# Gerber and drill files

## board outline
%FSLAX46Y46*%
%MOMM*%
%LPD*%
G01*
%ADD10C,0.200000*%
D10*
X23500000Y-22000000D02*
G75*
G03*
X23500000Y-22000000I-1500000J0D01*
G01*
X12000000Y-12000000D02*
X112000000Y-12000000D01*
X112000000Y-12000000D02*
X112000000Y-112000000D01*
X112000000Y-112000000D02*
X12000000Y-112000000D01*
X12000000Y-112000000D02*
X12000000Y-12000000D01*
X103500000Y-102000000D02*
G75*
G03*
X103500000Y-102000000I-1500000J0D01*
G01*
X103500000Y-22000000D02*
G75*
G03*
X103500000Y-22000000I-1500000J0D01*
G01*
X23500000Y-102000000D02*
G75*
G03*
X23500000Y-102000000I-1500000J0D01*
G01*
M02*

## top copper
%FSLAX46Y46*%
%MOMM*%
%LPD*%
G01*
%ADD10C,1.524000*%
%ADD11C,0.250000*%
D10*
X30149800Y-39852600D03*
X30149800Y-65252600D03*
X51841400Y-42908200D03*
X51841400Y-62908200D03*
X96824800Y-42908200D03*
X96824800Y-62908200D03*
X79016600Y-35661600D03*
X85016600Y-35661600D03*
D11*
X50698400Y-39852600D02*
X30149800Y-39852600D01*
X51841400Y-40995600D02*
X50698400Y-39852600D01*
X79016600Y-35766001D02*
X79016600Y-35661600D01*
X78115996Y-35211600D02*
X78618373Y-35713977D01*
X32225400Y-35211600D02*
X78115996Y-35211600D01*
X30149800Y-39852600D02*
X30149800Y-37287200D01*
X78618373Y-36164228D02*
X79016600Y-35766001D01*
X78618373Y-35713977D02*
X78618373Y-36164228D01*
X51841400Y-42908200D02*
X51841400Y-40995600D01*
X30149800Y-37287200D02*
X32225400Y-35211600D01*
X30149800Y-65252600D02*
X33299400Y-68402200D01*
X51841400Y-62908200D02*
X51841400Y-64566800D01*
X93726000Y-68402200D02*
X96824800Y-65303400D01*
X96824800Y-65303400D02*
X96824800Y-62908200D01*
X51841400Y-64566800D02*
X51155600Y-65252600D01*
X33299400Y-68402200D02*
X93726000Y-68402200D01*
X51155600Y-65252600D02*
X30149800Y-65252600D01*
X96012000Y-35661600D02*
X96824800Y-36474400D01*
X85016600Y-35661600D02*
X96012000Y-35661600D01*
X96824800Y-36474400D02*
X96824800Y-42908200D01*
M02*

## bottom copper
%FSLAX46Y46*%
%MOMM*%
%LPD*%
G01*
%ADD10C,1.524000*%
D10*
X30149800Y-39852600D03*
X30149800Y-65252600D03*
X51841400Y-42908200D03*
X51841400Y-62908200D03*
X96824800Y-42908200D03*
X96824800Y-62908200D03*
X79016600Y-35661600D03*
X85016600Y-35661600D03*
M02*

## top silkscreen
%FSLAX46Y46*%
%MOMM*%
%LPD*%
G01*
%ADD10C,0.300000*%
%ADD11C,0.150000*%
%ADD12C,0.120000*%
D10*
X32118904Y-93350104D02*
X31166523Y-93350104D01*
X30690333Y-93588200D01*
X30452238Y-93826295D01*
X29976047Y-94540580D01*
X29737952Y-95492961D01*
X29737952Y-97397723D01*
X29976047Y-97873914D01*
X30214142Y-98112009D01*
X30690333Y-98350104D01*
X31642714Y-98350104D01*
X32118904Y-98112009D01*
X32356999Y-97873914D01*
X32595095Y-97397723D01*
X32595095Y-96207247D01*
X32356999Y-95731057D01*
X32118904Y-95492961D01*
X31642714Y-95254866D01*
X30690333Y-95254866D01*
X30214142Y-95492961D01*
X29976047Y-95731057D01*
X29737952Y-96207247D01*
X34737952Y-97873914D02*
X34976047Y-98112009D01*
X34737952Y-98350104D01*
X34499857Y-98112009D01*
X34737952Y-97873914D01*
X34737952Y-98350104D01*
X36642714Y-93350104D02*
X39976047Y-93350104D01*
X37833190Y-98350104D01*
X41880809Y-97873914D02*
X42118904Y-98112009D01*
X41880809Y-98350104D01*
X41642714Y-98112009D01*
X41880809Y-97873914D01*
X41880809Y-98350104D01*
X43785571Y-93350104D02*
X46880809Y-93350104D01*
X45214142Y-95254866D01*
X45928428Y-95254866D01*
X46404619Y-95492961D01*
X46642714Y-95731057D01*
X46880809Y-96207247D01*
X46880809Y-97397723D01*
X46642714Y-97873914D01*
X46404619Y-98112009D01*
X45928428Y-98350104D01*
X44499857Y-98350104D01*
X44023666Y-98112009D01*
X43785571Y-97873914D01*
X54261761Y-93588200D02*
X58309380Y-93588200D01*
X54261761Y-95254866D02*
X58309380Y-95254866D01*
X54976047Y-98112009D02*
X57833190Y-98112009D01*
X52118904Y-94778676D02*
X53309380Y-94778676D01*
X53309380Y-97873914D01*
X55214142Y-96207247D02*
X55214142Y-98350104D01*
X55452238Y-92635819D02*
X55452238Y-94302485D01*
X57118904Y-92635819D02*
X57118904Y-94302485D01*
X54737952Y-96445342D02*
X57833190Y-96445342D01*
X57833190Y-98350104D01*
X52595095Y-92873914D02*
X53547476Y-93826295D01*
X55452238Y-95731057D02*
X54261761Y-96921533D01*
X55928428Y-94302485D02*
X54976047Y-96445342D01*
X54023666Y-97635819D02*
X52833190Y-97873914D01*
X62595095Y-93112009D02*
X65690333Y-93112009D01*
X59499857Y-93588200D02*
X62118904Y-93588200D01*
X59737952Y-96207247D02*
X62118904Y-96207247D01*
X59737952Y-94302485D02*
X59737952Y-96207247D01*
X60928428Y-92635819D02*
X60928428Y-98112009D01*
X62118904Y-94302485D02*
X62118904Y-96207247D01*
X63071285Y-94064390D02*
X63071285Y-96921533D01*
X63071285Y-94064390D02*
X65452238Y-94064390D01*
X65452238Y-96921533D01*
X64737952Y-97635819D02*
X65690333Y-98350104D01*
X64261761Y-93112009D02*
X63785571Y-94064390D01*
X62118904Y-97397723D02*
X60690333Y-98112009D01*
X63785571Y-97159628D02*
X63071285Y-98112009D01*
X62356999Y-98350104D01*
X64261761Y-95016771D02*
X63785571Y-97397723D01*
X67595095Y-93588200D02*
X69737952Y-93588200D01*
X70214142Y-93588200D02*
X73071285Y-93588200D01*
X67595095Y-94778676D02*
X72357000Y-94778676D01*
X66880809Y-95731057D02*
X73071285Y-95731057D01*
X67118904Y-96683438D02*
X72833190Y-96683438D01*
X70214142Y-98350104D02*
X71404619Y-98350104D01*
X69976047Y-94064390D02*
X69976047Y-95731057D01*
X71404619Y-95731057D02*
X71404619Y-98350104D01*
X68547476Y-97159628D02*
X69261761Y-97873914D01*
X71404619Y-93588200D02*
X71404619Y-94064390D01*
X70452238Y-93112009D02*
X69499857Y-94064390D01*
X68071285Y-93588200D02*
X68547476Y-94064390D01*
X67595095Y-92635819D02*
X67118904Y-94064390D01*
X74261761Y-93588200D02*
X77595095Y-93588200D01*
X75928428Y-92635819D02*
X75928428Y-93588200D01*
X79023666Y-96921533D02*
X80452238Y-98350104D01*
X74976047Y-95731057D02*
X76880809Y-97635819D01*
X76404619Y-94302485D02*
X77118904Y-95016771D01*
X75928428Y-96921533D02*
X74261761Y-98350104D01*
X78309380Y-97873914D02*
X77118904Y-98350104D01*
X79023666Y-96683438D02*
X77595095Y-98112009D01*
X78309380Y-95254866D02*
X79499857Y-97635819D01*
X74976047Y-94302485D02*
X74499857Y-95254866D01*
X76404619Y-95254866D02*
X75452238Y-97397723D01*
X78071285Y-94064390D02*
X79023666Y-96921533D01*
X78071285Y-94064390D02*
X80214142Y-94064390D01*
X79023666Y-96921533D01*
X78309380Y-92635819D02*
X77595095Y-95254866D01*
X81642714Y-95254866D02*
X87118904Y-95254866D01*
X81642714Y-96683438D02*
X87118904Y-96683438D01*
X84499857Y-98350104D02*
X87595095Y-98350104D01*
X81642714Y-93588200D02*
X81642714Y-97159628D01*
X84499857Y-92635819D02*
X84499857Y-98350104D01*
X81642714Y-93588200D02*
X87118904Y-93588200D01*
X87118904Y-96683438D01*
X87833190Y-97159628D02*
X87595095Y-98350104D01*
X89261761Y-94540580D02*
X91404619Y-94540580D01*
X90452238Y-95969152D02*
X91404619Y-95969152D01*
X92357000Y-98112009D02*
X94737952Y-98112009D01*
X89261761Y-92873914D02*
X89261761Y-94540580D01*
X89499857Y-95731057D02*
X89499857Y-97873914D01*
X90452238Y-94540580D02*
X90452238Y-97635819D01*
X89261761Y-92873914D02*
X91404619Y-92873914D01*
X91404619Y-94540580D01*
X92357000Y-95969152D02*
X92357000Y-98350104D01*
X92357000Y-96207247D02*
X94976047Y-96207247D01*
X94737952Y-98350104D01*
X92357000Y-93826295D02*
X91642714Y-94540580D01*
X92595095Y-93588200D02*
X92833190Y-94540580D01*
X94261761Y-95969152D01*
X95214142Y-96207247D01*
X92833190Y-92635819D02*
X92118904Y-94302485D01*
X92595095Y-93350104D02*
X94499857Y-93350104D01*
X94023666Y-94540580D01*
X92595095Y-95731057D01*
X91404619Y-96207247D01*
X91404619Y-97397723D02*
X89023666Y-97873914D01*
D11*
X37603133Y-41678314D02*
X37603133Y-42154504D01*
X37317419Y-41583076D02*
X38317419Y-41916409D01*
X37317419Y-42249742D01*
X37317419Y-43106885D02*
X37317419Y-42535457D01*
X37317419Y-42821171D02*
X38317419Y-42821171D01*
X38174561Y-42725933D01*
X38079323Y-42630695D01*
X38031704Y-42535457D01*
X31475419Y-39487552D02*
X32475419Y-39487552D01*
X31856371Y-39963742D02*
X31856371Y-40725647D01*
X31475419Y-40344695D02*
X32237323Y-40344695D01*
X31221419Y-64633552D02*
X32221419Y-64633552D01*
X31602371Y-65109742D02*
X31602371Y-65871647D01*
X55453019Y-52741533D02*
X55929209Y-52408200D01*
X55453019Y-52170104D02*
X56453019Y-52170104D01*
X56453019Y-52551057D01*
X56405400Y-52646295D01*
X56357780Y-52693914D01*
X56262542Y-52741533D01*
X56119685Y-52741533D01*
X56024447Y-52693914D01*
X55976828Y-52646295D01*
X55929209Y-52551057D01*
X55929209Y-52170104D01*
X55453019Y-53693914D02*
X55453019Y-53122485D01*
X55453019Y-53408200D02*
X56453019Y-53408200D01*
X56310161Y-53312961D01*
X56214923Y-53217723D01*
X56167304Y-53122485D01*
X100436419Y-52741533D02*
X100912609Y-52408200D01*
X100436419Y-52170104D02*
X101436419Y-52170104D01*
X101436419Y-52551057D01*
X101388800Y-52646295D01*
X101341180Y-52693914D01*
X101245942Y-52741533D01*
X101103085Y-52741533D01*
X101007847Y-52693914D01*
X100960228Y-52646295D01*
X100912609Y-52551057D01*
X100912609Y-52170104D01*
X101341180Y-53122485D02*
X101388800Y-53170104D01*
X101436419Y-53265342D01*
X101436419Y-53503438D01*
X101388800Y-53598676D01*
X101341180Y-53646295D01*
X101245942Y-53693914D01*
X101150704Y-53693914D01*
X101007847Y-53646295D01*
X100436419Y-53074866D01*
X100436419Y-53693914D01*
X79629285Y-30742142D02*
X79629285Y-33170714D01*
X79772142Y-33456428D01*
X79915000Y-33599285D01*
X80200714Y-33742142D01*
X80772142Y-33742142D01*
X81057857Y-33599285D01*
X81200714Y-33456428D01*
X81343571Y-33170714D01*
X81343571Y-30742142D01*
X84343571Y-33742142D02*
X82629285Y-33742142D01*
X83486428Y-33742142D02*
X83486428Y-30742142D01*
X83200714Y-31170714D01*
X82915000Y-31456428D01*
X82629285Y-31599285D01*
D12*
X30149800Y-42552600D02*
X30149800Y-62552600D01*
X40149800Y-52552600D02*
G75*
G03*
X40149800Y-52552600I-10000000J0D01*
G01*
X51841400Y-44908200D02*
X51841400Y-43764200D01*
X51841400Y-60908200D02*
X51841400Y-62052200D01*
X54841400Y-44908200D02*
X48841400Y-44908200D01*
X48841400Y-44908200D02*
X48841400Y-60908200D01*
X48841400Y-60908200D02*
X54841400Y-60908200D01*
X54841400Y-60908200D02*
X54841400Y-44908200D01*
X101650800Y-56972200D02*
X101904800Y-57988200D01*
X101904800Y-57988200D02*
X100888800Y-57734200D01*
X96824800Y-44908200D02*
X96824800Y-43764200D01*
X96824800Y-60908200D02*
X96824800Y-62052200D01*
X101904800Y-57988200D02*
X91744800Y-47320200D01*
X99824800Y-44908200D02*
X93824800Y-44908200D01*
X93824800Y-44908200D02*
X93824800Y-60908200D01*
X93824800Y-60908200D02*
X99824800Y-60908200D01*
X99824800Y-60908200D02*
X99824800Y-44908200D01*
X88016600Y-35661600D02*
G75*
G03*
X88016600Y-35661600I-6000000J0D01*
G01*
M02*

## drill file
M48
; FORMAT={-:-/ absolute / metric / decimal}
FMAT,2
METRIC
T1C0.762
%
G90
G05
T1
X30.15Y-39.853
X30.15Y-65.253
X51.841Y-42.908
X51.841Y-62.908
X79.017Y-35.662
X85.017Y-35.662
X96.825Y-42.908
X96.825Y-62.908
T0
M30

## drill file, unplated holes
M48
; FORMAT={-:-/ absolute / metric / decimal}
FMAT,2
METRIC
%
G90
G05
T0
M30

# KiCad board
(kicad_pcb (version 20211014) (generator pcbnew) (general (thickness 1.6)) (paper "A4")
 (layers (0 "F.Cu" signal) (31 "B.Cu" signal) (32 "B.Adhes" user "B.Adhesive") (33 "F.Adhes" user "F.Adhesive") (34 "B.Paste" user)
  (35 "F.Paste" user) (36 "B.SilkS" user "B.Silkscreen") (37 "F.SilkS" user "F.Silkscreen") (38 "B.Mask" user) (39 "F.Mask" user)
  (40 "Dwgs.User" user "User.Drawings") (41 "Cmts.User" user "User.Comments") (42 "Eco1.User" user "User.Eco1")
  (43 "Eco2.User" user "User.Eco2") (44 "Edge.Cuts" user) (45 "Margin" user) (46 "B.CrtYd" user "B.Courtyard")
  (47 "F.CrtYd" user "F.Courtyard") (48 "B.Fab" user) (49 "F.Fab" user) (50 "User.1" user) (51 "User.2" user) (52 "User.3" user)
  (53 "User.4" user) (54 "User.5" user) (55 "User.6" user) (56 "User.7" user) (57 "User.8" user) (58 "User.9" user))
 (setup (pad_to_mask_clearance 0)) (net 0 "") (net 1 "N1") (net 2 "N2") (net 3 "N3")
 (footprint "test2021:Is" (layer "F.Cu") (at 30.1498 52.5526 -90)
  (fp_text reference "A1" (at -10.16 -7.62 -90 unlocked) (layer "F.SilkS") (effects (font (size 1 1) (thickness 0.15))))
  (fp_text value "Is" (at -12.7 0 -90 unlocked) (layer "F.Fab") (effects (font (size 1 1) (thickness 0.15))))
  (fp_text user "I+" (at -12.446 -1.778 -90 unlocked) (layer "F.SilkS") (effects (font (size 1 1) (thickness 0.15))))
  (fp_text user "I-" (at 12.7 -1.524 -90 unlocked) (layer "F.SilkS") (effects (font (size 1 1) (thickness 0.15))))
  (fp_line (start -10 0) (end 10 0) (layer "F.SilkS") (width 0.12))
  (fp_circle (center 0 0) (end 10 0) (layer "F.SilkS") (width 0.12) (fill none))
  (pad "1" thru_hole circle (at -12.7 0 270) (size 1.524 1.524) (drill 0.762) (layers *.Cu *.Mask) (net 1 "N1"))
  (pad "2" thru_hole circle (at 12.7 0 270) (size 1.524 1.524) (drill 0.762) (layers *.Cu *.Mask) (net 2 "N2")))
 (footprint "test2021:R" (layer "F.Cu") (at 51.8414 52.9082 -90)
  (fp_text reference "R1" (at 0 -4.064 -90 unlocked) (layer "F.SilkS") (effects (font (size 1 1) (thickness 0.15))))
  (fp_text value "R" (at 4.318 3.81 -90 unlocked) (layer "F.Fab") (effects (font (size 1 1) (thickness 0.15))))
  (fp_line (start -8 0) (end -9.144 0) (layer "F.SilkS") (width 0.12))
  (fp_line (start 8 0) (end 9.144 0) (layer "F.SilkS") (width 0.12))
  (fp_rect (start -8 -3) (end 8 3) (layer "F.SilkS") (width 0.12) (fill none))
  (pad "1" thru_hole circle (at -10 0 270) (size 1.524 1.524) (drill 0.762) (layers *.Cu *.Mask) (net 1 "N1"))
  (pad "2" thru_hole circle (at 10 0 270) (size 1.524 1.524) (drill 0.762) (layers *.Cu *.Mask) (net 2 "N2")))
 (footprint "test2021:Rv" (layer "F.Cu") (at 96.8248 52.9082 -90)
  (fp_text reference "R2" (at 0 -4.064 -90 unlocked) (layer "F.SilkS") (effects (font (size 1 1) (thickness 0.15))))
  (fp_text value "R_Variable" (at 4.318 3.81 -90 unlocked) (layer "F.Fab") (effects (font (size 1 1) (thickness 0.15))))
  (fp_line (start 4.064 -4.826) (end 5.08 -5.08) (layer "F.SilkS") (width 0.12))
  (fp_line (start 5.08 -5.08) (end 4.826 -4.064) (layer "F.SilkS") (width 0.12))
  (fp_line (start -8 0) (end -9.144 0) (layer "F.SilkS") (width 0.12))
  (fp_line (start 8 0) (end 9.144 0) (layer "F.SilkS") (width 0.12))
  (fp_line (start 5.08 -5.08) (end -5.588 5.08) (layer "F.SilkS") (width 0.12))
  (fp_rect (start -8 -3) (end 8 3) (layer "F.SilkS") (width 0.12) (fill none))
  (pad "1" thru_hole circle (at -10 0 270) (size 1.524 1.524) (drill 0.762) (layers *.Cu *.Mask) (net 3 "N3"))
  (pad "2" thru_hole circle (at 10 0 270) (size 1.524 1.524) (drill 0.762) (layers *.Cu *.Mask) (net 2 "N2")))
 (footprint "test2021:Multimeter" (layer "F.Cu") (at 82.0166 35.6616 90)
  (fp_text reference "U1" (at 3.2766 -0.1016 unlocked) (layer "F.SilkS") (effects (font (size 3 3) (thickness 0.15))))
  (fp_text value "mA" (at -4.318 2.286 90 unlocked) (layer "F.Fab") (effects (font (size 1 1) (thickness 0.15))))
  (fp_circle (center 0 0) (end 6 0) (layer "F.SilkS") (width 0.12) (fill none))
  (pad "1" thru_hole circle (at 0 -3 90) (size 1.524 1.524) (drill 0.762) (layers *.Cu *.Mask) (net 1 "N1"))
  (pad "2" thru_hole circle (at 0 3 90) (size 1.524 1.524) (drill 0.762) (layers *.Cu *.Mask) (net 3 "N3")))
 (gr_circle (center 22 22) (end 23.5 22) (layer "Edge.Cuts") (width 0.2) (fill none))
 (gr_rect (start 12 12) (end 112 112) (layer "Edge.Cuts") (width 0.2) (fill none))
 (gr_circle (center 102 102) (end 103.5 102) (layer "Edge.Cuts") (width 0.2) (fill none))
 (gr_circle (center 102 22) (end 103.5 22) (layer "Edge.Cuts") (width 0.2) (fill none))
 (gr_circle (center 22 102) (end 23.5 102) (layer "Edge.Cuts") (width 0.2) (fill none))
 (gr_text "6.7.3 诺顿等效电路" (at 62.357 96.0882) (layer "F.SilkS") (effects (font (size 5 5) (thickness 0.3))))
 (segment (start 50.6984 39.8526) (end 30.1498 39.8526) (width 0.25) (layer "F.Cu") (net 1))
 (segment (start 51.8414 40.9956) (end 50.6984 39.8526) (width 0.25) (layer "F.Cu") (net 1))
 (segment (start 79.0166 35.766001) (end 79.0166 35.6616) (width 0.25) (layer "F.Cu") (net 1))
 (segment (start 78.115996 35.2116) (end 78.618373 35.713977) (width 0.25) (layer "F.Cu") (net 1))
 (segment (start 32.2254 35.2116) (end 78.115996 35.2116) (width 0.25) (layer "F.Cu") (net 1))
 (segment (start 30.1498 39.8526) (end 30.1498 37.2872) (width 0.25) (layer "F.Cu") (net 1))
 (segment (start 78.618373 36.164228) (end 79.0166 35.766001) (width 0.25) (layer "F.Cu") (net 1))
 (segment (start 78.618373 35.713977) (end 78.618373 36.164228) (width 0.25) (layer "F.Cu") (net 1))
 (segment (start 51.8414 42.9082) (end 51.8414 40.9956) (width 0.25) (layer "F.Cu") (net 1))
 (segment (start 30.1498 37.2872) (end 32.2254 35.2116) (width 0.25) (layer "F.Cu") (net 1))
 (segment (start 30.1498 65.2526) (end 33.2994 68.4022) (width 0.25) (layer "F.Cu") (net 2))
 (segment (start 51.8414 62.9082) (end 51.8414 64.5668) (width 0.25) (layer "F.Cu") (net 2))
 (segment (start 93.726 68.4022) (end 96.8248 65.3034) (width 0.25) (layer "F.Cu") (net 2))
 (segment (start 96.8248 65.3034) (end 96.8248 62.9082) (width 0.25) (layer "F.Cu") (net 2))
 (segment (start 51.8414 64.5668) (end 51.1556 65.2526) (width 0.25) (layer "F.Cu") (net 2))
 (segment (start 33.2994 68.4022) (end 93.726 68.4022) (width 0.25) (layer "F.Cu") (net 2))
 (segment (start 51.1556 65.2526) (end 30.1498 65.2526) (width 0.25) (layer "F.Cu") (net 2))
 (segment (start 96.012 35.6616) (end 96.8248 36.4744) (width 0.25) (layer "F.Cu") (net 3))
 (segment (start 85.0166 35.6616) (end 96.012 35.6616) (width 0.25) (layer "F.Cu") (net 3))
 (segment (start 96.8248 36.4744) (end 96.8248 42.9082) (width 0.25) (layer "F.Cu") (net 3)))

